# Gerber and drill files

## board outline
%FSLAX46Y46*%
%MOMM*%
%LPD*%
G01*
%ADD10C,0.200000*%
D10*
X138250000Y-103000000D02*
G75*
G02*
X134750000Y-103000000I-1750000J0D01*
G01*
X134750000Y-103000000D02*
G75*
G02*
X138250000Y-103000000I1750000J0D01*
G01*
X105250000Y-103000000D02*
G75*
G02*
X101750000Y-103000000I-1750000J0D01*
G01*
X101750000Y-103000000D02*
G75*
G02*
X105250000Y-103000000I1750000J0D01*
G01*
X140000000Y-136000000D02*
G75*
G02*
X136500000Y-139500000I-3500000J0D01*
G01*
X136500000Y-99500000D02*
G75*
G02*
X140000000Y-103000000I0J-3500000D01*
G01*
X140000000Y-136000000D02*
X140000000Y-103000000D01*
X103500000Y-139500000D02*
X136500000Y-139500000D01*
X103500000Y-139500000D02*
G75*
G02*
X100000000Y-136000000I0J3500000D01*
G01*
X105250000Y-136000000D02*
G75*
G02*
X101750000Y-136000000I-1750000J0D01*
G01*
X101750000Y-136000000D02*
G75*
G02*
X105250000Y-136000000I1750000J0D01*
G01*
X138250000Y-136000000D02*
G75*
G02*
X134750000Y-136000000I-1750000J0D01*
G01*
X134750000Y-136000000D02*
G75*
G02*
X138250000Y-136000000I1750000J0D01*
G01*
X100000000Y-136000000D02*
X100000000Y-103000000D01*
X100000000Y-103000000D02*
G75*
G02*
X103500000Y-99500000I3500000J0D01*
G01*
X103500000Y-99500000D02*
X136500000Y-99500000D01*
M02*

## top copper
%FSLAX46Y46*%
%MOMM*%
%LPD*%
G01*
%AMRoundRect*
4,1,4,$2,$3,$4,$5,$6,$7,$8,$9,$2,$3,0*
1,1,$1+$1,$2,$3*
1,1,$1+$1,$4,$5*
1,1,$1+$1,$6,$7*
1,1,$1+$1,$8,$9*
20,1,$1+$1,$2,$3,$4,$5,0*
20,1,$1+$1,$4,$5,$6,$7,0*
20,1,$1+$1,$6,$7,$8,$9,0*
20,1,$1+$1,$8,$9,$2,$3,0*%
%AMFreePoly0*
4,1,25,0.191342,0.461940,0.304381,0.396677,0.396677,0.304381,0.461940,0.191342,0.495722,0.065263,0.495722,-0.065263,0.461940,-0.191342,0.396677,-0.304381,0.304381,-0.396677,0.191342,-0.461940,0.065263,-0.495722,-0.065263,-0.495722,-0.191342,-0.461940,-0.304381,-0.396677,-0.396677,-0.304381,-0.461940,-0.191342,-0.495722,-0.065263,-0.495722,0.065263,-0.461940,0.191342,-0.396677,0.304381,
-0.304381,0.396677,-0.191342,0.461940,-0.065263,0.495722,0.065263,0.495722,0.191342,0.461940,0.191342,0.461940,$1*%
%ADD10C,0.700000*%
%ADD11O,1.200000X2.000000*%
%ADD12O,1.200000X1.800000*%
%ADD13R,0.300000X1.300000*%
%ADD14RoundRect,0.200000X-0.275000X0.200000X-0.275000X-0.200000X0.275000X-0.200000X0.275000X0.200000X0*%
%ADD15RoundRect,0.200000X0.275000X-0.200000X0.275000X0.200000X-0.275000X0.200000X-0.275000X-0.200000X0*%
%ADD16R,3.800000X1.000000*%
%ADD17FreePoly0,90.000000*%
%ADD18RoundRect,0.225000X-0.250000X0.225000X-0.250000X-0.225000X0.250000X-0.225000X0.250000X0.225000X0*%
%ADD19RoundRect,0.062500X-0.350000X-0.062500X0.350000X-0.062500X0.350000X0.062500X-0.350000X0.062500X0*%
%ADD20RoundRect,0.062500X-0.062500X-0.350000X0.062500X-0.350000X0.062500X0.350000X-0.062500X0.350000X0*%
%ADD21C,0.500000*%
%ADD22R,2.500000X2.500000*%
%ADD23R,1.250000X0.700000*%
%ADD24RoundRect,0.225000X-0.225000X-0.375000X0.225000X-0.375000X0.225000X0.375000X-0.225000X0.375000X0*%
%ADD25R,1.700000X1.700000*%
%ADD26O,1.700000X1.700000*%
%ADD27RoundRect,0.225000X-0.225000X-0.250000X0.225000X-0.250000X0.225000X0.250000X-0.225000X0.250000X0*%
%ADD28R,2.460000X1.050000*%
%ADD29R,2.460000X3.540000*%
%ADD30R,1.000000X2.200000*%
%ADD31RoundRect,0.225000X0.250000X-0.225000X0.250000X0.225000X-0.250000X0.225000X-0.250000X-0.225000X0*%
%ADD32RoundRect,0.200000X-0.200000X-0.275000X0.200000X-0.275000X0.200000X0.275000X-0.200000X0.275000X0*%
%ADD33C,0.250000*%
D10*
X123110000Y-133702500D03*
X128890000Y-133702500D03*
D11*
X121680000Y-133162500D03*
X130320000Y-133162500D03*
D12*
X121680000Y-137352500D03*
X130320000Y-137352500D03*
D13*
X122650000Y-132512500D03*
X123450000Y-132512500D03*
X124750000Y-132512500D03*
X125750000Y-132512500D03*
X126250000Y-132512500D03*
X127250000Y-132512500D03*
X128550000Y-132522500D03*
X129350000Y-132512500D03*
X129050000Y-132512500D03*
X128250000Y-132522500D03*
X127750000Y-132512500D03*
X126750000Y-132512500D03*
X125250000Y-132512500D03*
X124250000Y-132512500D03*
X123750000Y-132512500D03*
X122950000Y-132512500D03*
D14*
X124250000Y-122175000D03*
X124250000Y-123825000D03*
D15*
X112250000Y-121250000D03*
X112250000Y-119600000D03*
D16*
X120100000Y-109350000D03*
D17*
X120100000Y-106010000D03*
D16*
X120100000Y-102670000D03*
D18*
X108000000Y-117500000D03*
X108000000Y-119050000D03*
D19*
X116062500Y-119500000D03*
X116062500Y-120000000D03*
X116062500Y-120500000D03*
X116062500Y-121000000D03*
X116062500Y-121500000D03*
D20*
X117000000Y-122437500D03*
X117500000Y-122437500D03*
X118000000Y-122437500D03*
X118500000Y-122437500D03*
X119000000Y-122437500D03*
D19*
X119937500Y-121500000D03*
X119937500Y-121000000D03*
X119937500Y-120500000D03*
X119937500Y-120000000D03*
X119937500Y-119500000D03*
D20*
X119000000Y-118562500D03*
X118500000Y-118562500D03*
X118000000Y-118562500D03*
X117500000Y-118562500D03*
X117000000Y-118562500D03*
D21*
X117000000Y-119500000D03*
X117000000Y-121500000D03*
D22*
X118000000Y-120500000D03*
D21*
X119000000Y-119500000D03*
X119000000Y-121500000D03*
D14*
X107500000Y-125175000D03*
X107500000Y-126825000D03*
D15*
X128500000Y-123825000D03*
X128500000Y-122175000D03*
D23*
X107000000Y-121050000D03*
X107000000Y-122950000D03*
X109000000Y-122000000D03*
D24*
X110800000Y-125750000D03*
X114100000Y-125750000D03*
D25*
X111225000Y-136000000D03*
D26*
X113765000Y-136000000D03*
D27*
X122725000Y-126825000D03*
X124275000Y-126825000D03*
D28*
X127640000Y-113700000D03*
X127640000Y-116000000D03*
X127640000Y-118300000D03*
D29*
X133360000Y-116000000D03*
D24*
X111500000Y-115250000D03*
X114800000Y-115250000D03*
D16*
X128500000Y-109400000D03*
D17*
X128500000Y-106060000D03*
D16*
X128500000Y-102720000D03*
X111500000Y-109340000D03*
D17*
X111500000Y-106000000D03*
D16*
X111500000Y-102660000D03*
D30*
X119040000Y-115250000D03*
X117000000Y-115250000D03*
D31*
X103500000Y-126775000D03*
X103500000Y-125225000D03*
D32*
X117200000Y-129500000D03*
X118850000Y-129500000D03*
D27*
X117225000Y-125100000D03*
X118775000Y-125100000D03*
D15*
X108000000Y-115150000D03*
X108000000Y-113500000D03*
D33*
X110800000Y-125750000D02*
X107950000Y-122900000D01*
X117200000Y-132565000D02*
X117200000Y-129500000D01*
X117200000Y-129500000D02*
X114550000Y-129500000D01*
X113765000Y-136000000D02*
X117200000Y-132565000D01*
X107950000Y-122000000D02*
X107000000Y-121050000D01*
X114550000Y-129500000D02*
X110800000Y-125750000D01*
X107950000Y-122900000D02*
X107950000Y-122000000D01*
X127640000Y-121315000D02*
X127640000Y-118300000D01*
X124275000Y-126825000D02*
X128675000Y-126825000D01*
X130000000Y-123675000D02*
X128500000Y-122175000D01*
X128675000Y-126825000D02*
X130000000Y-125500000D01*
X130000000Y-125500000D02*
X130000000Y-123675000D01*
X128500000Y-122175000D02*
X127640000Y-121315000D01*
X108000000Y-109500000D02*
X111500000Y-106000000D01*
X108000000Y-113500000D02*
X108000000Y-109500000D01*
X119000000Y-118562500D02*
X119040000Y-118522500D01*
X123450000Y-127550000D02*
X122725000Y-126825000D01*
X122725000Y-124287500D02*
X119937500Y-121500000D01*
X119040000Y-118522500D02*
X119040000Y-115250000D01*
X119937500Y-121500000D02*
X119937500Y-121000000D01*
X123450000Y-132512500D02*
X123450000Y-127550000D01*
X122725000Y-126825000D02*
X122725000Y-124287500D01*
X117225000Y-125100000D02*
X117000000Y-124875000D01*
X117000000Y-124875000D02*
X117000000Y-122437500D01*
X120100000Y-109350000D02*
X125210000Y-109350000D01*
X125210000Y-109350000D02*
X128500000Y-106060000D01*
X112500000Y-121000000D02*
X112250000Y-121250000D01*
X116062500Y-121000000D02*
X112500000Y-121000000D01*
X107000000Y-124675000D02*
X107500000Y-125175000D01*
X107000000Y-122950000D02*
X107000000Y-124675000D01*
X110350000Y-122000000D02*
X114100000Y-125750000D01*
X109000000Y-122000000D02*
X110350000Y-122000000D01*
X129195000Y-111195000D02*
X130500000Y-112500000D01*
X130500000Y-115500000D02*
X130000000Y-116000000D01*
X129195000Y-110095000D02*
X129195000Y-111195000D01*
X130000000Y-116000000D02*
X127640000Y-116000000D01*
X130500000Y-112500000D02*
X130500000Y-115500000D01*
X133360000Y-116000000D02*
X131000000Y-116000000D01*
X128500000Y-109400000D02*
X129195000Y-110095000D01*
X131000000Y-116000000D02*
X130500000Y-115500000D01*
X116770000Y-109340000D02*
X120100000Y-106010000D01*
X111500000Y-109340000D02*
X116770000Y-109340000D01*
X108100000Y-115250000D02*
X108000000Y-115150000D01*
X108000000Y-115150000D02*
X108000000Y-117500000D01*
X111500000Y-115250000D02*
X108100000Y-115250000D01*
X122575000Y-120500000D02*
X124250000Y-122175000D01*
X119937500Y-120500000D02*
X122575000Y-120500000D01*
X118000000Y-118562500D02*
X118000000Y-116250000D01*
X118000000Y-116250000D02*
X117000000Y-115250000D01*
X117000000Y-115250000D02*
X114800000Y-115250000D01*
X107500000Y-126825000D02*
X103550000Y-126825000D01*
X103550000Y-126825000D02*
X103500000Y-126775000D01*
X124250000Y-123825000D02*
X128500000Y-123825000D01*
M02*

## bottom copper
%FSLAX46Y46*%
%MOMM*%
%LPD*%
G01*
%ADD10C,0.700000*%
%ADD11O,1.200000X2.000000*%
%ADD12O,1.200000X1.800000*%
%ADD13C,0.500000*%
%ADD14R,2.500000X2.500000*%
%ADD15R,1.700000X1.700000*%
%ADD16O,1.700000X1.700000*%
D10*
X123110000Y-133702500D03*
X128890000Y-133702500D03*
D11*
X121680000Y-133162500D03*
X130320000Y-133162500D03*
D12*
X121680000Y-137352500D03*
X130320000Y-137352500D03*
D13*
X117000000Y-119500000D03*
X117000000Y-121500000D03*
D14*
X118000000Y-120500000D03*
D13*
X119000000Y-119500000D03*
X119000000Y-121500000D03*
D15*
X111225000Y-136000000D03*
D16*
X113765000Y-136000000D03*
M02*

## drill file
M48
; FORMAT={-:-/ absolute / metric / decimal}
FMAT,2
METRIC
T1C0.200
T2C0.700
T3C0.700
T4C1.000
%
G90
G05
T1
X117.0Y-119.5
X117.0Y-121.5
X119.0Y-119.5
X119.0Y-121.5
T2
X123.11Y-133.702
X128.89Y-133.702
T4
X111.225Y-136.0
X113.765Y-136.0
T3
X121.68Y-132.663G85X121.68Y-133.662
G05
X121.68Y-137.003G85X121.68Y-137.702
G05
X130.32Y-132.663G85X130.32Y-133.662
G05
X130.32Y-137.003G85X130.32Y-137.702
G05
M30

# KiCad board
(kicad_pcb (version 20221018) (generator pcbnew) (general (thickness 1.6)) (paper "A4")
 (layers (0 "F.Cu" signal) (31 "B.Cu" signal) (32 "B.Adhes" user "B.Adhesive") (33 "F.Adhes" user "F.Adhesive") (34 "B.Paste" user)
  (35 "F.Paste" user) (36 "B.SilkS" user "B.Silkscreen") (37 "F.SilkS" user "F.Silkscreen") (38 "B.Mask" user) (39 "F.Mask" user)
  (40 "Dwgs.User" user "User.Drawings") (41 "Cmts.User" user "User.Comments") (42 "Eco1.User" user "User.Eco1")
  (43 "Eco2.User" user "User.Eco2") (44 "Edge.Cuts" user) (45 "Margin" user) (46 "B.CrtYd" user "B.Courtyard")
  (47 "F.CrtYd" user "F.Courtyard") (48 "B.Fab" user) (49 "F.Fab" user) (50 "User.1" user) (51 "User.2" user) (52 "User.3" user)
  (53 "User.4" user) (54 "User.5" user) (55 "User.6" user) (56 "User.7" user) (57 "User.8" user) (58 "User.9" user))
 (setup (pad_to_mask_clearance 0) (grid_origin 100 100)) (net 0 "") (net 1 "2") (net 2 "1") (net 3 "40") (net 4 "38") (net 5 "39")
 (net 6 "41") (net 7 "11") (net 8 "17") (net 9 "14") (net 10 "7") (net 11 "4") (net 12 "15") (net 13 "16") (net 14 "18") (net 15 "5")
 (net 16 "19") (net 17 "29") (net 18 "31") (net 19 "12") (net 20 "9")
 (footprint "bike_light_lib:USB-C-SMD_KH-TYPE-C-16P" (layer "F.Cu") (at 126 134.9325)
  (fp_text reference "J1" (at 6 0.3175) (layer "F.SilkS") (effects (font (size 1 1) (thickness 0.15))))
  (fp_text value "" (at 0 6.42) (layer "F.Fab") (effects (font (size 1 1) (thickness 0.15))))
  (pad "" thru_hole circle (at -2.89 -1.23) (size 0.7 0.7) (drill 0.7) (layers "*.Cu" "*.Mask"))
  (pad "" thru_hole circle (at 2.89 -1.23) (size 0.7 0.7) (drill 0.7) (layers "*.Cu" "*.Mask"))
  (pad "1" thru_hole oval (at -4.32 -1.77) (size 1.2 2) (drill oval 0.700024 1.699997) (layers "*.Cu" "*.Paste" "*.Mask") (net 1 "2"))
  (pad "2" thru_hole oval (at 4.32 -1.77) (size 1.2 2) (drill oval 0.700024 1.699997) (layers "*.Cu" "*.Paste" "*.Mask") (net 1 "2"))
  (pad "3" thru_hole oval (at -4.32 2.42) (size 1.2 1.8) (drill oval 0.700024 1.399997) (layers "*.Cu" "*.Paste" "*.Mask") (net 1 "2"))
  (pad "4" thru_hole oval (at 4.32 2.42) (size 1.2 1.8) (drill oval 0.700024 1.399997) (layers "*.Cu" "*.Paste" "*.Mask") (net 1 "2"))
  (pad "A1" smd rect (at -3.35 -2.42) (size 0.3 1.3) (layers "F.Cu" "F.Paste" "F.Mask") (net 1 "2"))
  (pad "A4" smd rect (at -2.55 -2.42) (size 0.3 1.3) (layers "F.Cu" "F.Paste" "F.Mask") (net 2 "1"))
  (pad "A5" smd rect (at -1.25 -2.42) (size 0.3 1.3) (layers "F.Cu" "F.Paste" "F.Mask") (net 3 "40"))
  (pad "A6" smd rect (at -0.25 -2.42) (size 0.3 1.3) (layers "F.Cu" "F.Paste" "F.Mask") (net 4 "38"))
  (pad "A7" smd rect (at 0.25 -2.42) (size 0.3 1.3) (layers "F.Cu" "F.Paste" "F.Mask") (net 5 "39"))
  (pad "A8" smd rect (at 1.25 -2.42) (size 0.3 1.3) (layers "F.Cu" "F.Paste" "F.Mask") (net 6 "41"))
  (pad "A9" smd rect (at 2.55 -2.41) (size 0.3 1.3) (layers "F.Cu" "F.Paste" "F.Mask") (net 2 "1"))
  (pad "A12" smd rect (at 3.35 -2.42) (size 0.3 1.3) (layers "F.Cu" "F.Paste" "F.Mask") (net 1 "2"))
  (pad "B1" smd rect (at 3.05 -2.42) (size 0.3 1.3) (layers "F.Cu" "F.Paste" "F.Mask") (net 1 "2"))
  (pad "B4" smd rect (at 2.25 -2.41) (size 0.3 1.3) (layers "F.Cu" "F.Paste" "F.Mask") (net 2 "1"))
  (pad "B5" smd rect (at 1.75 -2.42) (size 0.3 1.3) (layers "F.Cu" "F.Paste" "F.Mask") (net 3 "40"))
  (pad "B6" smd rect (at 0.75 -2.42) (size 0.3 1.3) (layers "F.Cu" "F.Paste" "F.Mask") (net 4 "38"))
  (pad "B7" smd rect (at -0.75 -2.42) (size 0.3 1.3) (layers "F.Cu" "F.Paste" "F.Mask") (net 5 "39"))
  (pad "B8" smd rect (at -1.75 -2.42) (size 0.3 1.3) (layers "F.Cu" "F.Paste" "F.Mask") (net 6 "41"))
  (pad "B9" smd rect (at -2.25 -2.42) (size 0.3 1.3) (layers "F.Cu" "F.Paste" "F.Mask") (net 2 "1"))
  (pad "B12" smd rect (at -3.05 -2.42) (size 0.3 1.3) (layers "F.Cu" "F.Paste" "F.Mask") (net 1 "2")))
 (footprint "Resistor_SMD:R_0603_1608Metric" (layer "F.Cu") (at 124.25 123 -90)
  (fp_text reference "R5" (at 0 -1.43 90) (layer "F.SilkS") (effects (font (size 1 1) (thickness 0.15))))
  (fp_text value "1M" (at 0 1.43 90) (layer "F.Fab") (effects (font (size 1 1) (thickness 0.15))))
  (pad "1" smd roundrect (at -0.825 0 270) (size 0.8 0.95) (layers "F.Cu" "F.Paste" "F.Mask") (roundrect_rratio 0.25) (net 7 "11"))
  (pad "2" smd roundrect (at 0.825 0 270) (size 0.8 0.95) (layers "F.Cu" "F.Paste" "F.Mask") (roundrect_rratio 0.25) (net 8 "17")))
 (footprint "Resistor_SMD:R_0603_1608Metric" (layer "F.Cu") (at 112.25 120.425 90)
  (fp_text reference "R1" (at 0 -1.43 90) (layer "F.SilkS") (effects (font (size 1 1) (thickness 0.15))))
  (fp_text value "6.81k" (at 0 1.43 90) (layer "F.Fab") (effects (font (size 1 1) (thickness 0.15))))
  (pad "1" smd roundrect (at -0.825 0 90) (size 0.8 0.95) (layers "F.Cu" "F.Paste" "F.Mask") (roundrect_rratio 0.25) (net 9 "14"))
  (pad "2" smd roundrect (at 0.825 0 90) (size 0.8 0.95) (layers "F.Cu" "F.Paste" "F.Mask") (roundrect_rratio 0.25) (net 1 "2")))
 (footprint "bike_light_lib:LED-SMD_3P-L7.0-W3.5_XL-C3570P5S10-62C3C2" (layer "F.Cu") (at 120.1 106.01 90)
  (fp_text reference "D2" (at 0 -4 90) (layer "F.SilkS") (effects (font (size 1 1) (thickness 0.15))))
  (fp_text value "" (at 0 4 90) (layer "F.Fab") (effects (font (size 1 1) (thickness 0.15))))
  (pad "1" smd rect (at -3.34 0 90) (size 1 3.8) (layers "F.Cu" "F.Paste" "F.Mask") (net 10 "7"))
  (pad "2" smd custom (at 0 0 90) (size 1 1) (layers "F.Cu" "F.Paste" "F.Mask") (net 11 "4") (thermal_bridge_angle 45)
   (options (clearance outline) (anchor circle)) (primitives))
  (pad "3" smd rect (at 3.34 0 90) (size 1 3.8) (layers "F.Cu" "F.Paste" "F.Mask")))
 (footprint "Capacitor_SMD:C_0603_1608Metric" (layer "F.Cu") (at 108 118.275 -90)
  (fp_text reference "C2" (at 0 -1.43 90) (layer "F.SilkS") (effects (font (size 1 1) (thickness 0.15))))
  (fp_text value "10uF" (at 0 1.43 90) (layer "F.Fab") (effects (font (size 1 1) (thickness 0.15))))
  (pad "1" smd roundrect (at -0.775 0 270) (size 0.9 0.95) (layers "F.Cu" "F.Paste" "F.Mask") (roundrect_rratio 0.25) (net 7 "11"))
  (pad "2" smd roundrect (at 0.775 0 270) (size 0.9 0.95) (layers "F.Cu" "F.Paste" "F.Mask") (roundrect_rratio 0.25) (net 1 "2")))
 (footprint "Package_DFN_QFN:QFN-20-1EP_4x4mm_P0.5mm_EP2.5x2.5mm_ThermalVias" (layer "F.Cu") (at 118 120.5)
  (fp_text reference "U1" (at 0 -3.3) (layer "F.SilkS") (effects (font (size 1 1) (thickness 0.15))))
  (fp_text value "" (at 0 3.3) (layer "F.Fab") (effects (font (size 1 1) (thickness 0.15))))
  (pad "" smd roundrect (at -0.625 -0.625) (size 1.08 1.08) (layers "F.Paste") (roundrect_rratio 0.231481))
  (pad "" smd roundrect (at -0.625 0.625) (size 1.08 1.08) (layers "F.Paste") (roundrect_rratio 0.231481))
  (pad "" smd roundrect (at 0.625 -0.625) (size 1.08 1.08) (layers "F.Paste") (roundrect_rratio 0.231481))
  (pad "" smd roundrect (at 0.625 0.625) (size 1.08 1.08) (layers "F.Paste") (roundrect_rratio 0.231481))
  (pad "1" smd roundrect (at -1.9375 -1) (size 0.825 0.25) (layers "F.Cu" "F.Paste" "F.Mask") (roundrect_rratio 0.25))
  (pad "2" smd roundrect (at -1.9375 -0.5) (size 0.825 0.25) (layers "F.Cu" "F.Paste" "F.Mask") (roundrect_rratio 0.25))
  (pad "3" smd roundrect (at -1.9375 0) (size 0.825 0.25) (layers "F.Cu" "F.Paste" "F.Mask") (roundrect_rratio 0.25) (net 2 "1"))
  (pad "4" smd roundrect (at -1.9375 0.5) (size 0.825 0.25) (layers "F.Cu" "F.Paste" "F.Mask") (roundrect_rratio 0.25) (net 9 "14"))
  (pad "5" smd roundrect (at -1.9375 1) (size 0.825 0.25) (layers "F.Cu" "F.Paste" "F.Mask") (roundrect_rratio 0.25) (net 2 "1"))
  (pad "6" smd roundrect (at -1 1.9375) (size 0.25 0.825) (layers "F.Cu" "F.Paste" "F.Mask") (roundrect_rratio 0.25) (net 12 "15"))
  (pad "7" smd roundrect (at -0.5 1.9375) (size 0.25 0.825) (layers "F.Cu" "F.Paste" "F.Mask") (roundrect_rratio 0.25) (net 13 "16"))
  (pad "8" smd roundrect (at 0 1.9375) (size 0.25 0.825) (layers "F.Cu" "F.Paste" "F.Mask") (roundrect_rratio 0.25) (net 8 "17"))
  (pad "9" smd roundrect (at 0.5 1.9375) (size 0.25 0.825) (layers "F.Cu" "F.Paste" "F.Mask") (roundrect_rratio 0.25) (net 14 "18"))
  (pad "10" smd roundrect (at 1 1.9375) (size 0.25 0.825) (layers "F.Cu" "F.Paste" "F.Mask") (roundrect_rratio 0.25) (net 14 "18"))
  (pad "11" smd roundrect (at 1.9375 1) (size 0.825 0.25) (layers "F.Cu" "F.Paste" "F.Mask") (roundrect_rratio 0.25) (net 2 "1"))
  (pad "12" smd roundrect (at 1.9375 0.5) (size 0.825 0.25) (layers "F.Cu" "F.Paste" "F.Mask") (roundrect_rratio 0.25) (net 2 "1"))
  (pad "13" smd roundrect (at 1.9375 0) (size 0.825 0.25) (layers "F.Cu" "F.Paste" "F.Mask") (roundrect_rratio 0.25) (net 7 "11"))
  (pad "14" smd roundrect (at 1.9375 -0.5) (size 0.825 0.25) (layers "F.Cu" "F.Paste" "F.Mask") (roundrect_rratio 0.25) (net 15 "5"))
  (pad "15" smd roundrect (at 1.9375 -1) (size 0.825 0.25) (layers "F.Cu" "F.Paste" "F.Mask") (roundrect_rratio 0.25) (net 2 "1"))
  (pad "16" smd roundrect (at 1 -1.9375) (size 0.25 0.825) (layers "F.Cu" "F.Paste" "F.Mask") (roundrect_rratio 0.25) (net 2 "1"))
  (pad "17" smd roundrect (at 0.5 -1.9375) (size 0.25 0.825) (layers "F.Cu" "F.Paste" "F.Mask") (roundrect_rratio 0.25) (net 1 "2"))
  (pad "18" smd roundrect (at 0 -1.9375) (size 0.25 0.825) (layers "F.Cu" "F.Paste" "F.Mask") (roundrect_rratio 0.25) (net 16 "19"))
  (pad "19" smd roundrect (at -0.5 -1.9375) (size 0.25 0.825) (layers "F.Cu" "F.Paste" "F.Mask") (roundrect_rratio 0.25))
  (pad "20" smd roundrect (at -1 -1.9375) (size 0.25 0.825) (layers "F.Cu" "F.Paste" "F.Mask") (roundrect_rratio 0.25))
  (pad "21" thru_hole circle (at -1 -1) (size 0.5 0.5) (drill 0.2) (layers "*.Cu"))
  (pad "21" thru_hole circle (at -1 1) (size 0.5 0.5) (drill 0.2) (layers "*.Cu"))
  (pad "21" smd rect (at 0 0) (size 2.5 2.5) (layers "F.Cu" "F.Mask")) (pad "21" smd rect (at 0 0) (size 2.5 2.5) (layers "B.Cu"))
  (pad "21" thru_hole circle (at 1 -1) (size 0.5 0.5) (drill 0.2) (layers "*.Cu"))
  (pad "21" thru_hole circle (at 1 1) (size 0.5 0.5) (drill 0.2) (layers "*.Cu")))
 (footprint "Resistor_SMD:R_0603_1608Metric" (layer "F.Cu") (at 107.5 126 -90)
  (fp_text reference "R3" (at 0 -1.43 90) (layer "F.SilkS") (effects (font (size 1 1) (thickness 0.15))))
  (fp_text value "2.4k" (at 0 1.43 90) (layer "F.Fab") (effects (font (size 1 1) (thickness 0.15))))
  (pad "1" smd roundrect (at -0.825 0 270) (size 0.8 0.95) (layers "F.Cu" "F.Paste" "F.Mask") (roundrect_rratio 0.25) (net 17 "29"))
  (pad "2" smd roundrect (at 0.825 0 270) (size 0.8 0.95) (layers "F.Cu" "F.Paste" "F.Mask") (roundrect_rratio 0.25) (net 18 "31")))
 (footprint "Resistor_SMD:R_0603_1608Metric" (layer "F.Cu") (at 128.5 123 90)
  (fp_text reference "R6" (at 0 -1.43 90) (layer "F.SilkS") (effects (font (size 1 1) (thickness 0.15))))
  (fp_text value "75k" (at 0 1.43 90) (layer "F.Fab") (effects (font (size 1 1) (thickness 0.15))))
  (pad "1" smd roundrect (at -0.825 0 90) (size 0.8 0.95) (layers "F.Cu" "F.Paste" "F.Mask") (roundrect_rratio 0.25) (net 8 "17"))
  (pad "2" smd roundrect (at 0.825 0 90) (size 0.8 0.95) (layers "F.Cu" "F.Paste" "F.Mask") (roundrect_rratio 0.25) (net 1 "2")))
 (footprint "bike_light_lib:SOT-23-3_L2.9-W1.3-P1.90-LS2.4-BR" (layer "F.Cu") (at 108 122 180)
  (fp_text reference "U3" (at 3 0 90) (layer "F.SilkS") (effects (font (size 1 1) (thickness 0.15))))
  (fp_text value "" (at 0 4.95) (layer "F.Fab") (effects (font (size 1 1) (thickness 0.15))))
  (pad "1" smd rect (at 1 0.95 180) (size 1.25 0.7) (layers "F.Cu" "F.Paste" "F.Mask") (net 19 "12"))
  (pad "2" smd rect (at 1 -0.95 180) (size 1.25 0.7) (layers "F.Cu" "F.Paste" "F.Mask") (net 17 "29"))
  (pad "3" smd rect (at -1 0 180) (size 1.25 0.7) (layers "F.Cu" "F.Paste" "F.Mask") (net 13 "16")))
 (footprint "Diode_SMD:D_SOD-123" (layer "F.Cu") (at 112.45 125.75)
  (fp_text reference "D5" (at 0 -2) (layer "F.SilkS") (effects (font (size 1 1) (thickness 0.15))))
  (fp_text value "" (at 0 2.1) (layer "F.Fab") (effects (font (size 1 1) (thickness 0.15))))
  (pad "1" smd roundrect (at -1.65 0) (size 0.9 1.2) (layers "F.Cu" "F.Paste" "F.Mask") (roundrect_rratio 0.25) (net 19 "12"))
  (pad "2" smd roundrect (at 1.65 0) (size 0.9 1.2) (layers "F.Cu" "F.Paste" "F.Mask") (roundrect_rratio 0.25) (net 13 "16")))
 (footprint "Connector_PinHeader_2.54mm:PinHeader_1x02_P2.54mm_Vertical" (layer "F.Cu") (at 111.225 136 90)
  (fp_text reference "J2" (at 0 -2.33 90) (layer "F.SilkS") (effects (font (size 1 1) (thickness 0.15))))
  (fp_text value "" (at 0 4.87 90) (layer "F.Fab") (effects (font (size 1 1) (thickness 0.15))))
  (pad "1" thru_hole rect (at 0 0 90) (size 1.7 1.7) (drill 1) (layers "*.Cu" "*.Mask") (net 1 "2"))
  (pad "2" thru_hole oval (at 0 2.54 90) (size 1.7 1.7) (drill 1) (layers "*.Cu" "*.Mask") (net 19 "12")))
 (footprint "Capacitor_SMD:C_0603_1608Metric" (layer "F.Cu") (at 123.5 126.825)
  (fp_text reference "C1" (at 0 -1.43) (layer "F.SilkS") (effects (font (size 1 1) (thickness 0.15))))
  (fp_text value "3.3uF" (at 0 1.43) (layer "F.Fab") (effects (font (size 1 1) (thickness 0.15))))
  (pad "1" smd roundrect (at -0.775 0) (size 0.9 0.95) (layers "F.Cu" "F.Paste" "F.Mask") (roundrect_rratio 0.25) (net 2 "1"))
  (pad "2" smd roundrect (at 0.775 0) (size 0.9 0.95) (layers "F.Cu" "F.Paste" "F.Mask") (roundrect_rratio 0.25) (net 1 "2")))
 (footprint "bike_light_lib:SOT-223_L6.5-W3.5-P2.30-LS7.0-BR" (layer "F.Cu") (at 130.5 116 180)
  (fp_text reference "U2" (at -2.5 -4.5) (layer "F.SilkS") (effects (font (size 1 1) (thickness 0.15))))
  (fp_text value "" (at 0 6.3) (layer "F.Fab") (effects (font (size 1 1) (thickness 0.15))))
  (pad "1" smd rect (at 2.86 2.3 180) (size 2.46 1.05) (layers "F.Cu" "F.Paste" "F.Mask") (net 19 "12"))
  (pad "2" smd rect (at 2.86 0 180) (size 2.46 1.05) (layers "F.Cu" "F.Paste" "F.Mask") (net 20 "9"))
  (pad "3" smd rect (at 2.86 -2.3 180) (size 2.46 1.05) (layers "F.Cu" "F.Paste" "F.Mask") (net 1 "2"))
  (pad "4" smd rect (at -2.86 0 180) (size 2.46 3.54) (layers "F.Cu" "F.Paste" "F.Mask") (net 20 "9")))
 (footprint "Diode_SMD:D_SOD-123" (layer "F.Cu") (at 113.15 115.25)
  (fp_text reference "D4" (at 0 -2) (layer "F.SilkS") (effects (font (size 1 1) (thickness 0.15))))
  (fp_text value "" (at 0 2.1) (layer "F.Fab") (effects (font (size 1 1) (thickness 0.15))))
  (pad "1" smd roundrect (at -1.65 0) (size 0.9 1.2) (layers "F.Cu" "F.Paste" "F.Mask") (roundrect_rratio 0.25) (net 7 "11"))
  (pad "2" smd roundrect (at 1.65 0) (size 0.9 1.2) (layers "F.Cu" "F.Paste" "F.Mask") (roundrect_rratio 0.25) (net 16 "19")))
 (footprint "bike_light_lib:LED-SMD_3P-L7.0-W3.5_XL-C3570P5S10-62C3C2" (layer "F.Cu") (at 128.5 106.06 90)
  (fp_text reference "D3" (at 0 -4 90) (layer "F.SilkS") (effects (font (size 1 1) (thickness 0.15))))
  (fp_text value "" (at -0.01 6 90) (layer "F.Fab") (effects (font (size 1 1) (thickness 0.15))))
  (pad "1" smd rect (at -3.34 0 90) (size 1 3.8) (layers "F.Cu" "F.Paste" "F.Mask") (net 20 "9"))
  (pad "2" smd custom (at 0 0 90) (size 1 1) (layers "F.Cu" "F.Paste" "F.Mask") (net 10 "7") (thermal_bridge_angle 45)
   (options (clearance outline) (anchor circle)) (primitives))
  (pad "3" smd rect (at 3.34 0 90) (size 1 3.8) (layers "F.Cu" "F.Paste" "F.Mask")))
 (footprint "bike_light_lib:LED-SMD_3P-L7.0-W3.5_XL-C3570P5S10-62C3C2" (layer "F.Cu") (at 111.5 106 90)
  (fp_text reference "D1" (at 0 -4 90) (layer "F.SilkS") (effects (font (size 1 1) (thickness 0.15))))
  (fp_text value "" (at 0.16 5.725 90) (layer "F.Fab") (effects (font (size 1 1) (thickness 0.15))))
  (pad "1" smd rect (at -3.34 0 90) (size 1 3.8) (layers "F.Cu" "F.Paste" "F.Mask") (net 11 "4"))
  (pad "2" smd custom (at 0 0 90) (size 1 1) (layers "F.Cu" "F.Paste" "F.Mask") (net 15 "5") (thermal_bridge_angle 45)
   (options (clearance outline) (anchor circle)) (primitives))
  (pad "3" smd rect (at 3.34 0 90) (size 1 3.8) (layers "F.Cu" "F.Paste" "F.Mask")))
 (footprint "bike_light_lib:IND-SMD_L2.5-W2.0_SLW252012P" (layer "F.Cu") (at 118.02 115.25 180)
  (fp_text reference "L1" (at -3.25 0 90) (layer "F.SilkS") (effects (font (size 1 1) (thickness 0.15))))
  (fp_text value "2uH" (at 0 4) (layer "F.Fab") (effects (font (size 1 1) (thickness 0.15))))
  (pad "1" smd rect (at -1.02 0 180) (size 1 2.2) (layers "F.Cu" "F.Paste" "F.Mask") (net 2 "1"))
  (pad "2" smd rect (at 1.02 0 180) (size 1 2.2) (layers "F.Cu" "F.Paste" "F.Mask") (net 16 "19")))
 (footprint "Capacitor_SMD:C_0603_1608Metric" (layer "F.Cu") (at 103.5 126 90)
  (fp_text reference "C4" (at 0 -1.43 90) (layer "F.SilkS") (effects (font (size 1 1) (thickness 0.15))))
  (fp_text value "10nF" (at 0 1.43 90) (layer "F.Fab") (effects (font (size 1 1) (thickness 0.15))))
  (pad "1" smd roundrect (at -0.775 0 90) (size 0.9 0.95) (layers "F.Cu" "F.Paste" "F.Mask") (roundrect_rratio 0.25) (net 18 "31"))
  (pad "2" smd roundrect (at 0.775 0 90) (size 0.9 0.95) (layers "F.Cu" "F.Paste" "F.Mask") (roundrect_rratio 0.25) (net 1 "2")))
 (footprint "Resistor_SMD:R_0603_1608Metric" (layer "F.Cu") (at 118.025 129.5)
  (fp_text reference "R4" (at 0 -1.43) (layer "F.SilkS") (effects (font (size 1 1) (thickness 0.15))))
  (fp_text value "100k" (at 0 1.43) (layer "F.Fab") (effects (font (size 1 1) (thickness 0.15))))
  (pad "1" smd roundrect (at -0.825 0) (size 0.8 0.95) (layers "F.Cu" "F.Paste" "F.Mask") (roundrect_rratio 0.25) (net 19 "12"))
  (pad "2" smd roundrect (at 0.825 0) (size 0.8 0.95) (layers "F.Cu" "F.Paste" "F.Mask") (roundrect_rratio 0.25) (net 1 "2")))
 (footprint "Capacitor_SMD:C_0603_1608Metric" (layer "F.Cu") (at 118 125.1)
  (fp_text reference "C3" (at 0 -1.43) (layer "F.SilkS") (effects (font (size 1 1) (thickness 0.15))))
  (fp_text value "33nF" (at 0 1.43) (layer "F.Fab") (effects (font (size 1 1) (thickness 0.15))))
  (pad "1" smd roundrect (at -0.775 0) (size 0.9 0.95) (layers "F.Cu" "F.Paste" "F.Mask") (roundrect_rratio 0.25) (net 12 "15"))
  (pad "2" smd roundrect (at 0.775 0) (size 0.9 0.95) (layers "F.Cu" "F.Paste" "F.Mask") (roundrect_rratio 0.25) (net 1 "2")))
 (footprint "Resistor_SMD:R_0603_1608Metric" (layer "F.Cu") (at 108 114.325 90)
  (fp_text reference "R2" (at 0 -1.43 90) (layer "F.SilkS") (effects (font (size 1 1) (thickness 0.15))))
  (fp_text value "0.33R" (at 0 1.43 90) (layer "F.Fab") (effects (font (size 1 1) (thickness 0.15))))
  (pad "1" smd roundrect (at -0.825 0 90) (size 0.8 0.95) (layers "F.Cu" "F.Paste" "F.Mask") (roundrect_rratio 0.25) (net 7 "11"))
  (pad "2" smd roundrect (at 0.825 0 90) (size 0.8 0.95) (layers "F.Cu" "F.Paste" "F.Mask") (roundrect_rratio 0.25) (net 15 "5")))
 (gr_circle (center 136.5 103) (end 138.25 103) (stroke (width 0.2) (type solid)) (fill none) (layer "Edge.Cuts"))
 (gr_circle (center 103.5 103) (end 105.25 103) (stroke (width 0.2) (type solid)) (fill none) (layer "Edge.Cuts"))
 (gr_arc (start 140 136) (mid 138.974874 138.474874) (end 136.5 139.5) (stroke (width 0.2) (type solid)) (layer "Edge.Cuts"))
 (gr_arc (start 136.5 99.5) (mid 138.974874 100.525126) (end 140 103) (stroke (width 0.2) (type solid)) (layer "Edge.Cuts"))
 (gr_line (start 140 136) (end 140 103) (stroke (width 0.2) (type solid)) (layer "Edge.Cuts"))
 (gr_line (start 103.5 139.5) (end 136.5 139.5) (stroke (width 0.2) (type solid)) (layer "Edge.Cuts"))
 (gr_arc (start 103.5 139.5) (mid 101.025126 138.474874) (end 100 136) (stroke (width 0.2) (type solid)) (layer "Edge.Cuts"))
 (gr_circle (center 103.5 136) (end 105.25 136) (stroke (width 0.2) (type solid)) (fill none) (layer "Edge.Cuts"))
 (gr_circle (center 136.5 136) (end 138.25 136) (stroke (width 0.2) (type solid)) (fill none) (layer "Edge.Cuts"))
 (gr_line (start 100 136) (end 100 103) (stroke (width 0.2) (type solid)) (layer "Edge.Cuts"))
 (gr_arc (start 100 103) (mid 101.025126 100.525126) (end 103.5 99.5) (stroke (width 0.2) (type solid)) (layer "Edge.Cuts"))
 (gr_line (start 103.5 99.5) (end 136.5 99.5) (stroke (width 0.2) (type solid)) (layer "Edge.Cuts"))
 (segment (start 110.8 125.75) (end 107.95 122.9) (width 0.25) (layer "F.Cu") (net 19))
 (segment (start 117.2 132.565) (end 117.2 129.5) (width 0.25) (layer "F.Cu") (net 19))
 (segment (start 117.2 129.5) (end 114.55 129.5) (width 0.25) (layer "F.Cu") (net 19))
 (segment (start 113.765 136) (end 117.2 132.565) (width 0.25) (layer "F.Cu") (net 19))
 (segment (start 107.95 122) (end 107 121.05) (width 0.25) (layer "F.Cu") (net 19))
 (segment (start 114.55 129.5) (end 110.8 125.75) (width 0.25) (layer "F.Cu") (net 19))
 (segment (start 107.95 122.9) (end 107.95 122) (width 0.25) (layer "F.Cu") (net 19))
 (segment (start 127.64 121.315) (end 127.64 118.3) (width 0.25) (layer "F.Cu") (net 1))
 (segment (start 124.275 126.825) (end 128.675 126.825) (width 0.25) (layer "F.Cu") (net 1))
 (segment (start 130 123.675) (end 128.5 122.175) (width 0.25) (layer "F.Cu") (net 1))
 (segment (start 128.675 126.825) (end 130 125.5) (width 0.25) (layer "F.Cu") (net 1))
 (segment (start 130 125.5) (end 130 123.675) (width 0.25) (layer "F.Cu") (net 1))
 (segment (start 128.5 122.175) (end 127.64 121.315) (width 0.25) (layer "F.Cu") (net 1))
 (segment (start 108 109.5) (end 111.5 106) (width 0.25) (layer "F.Cu") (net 15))
 (segment (start 108 113.5) (end 108 109.5) (width 0.25) (layer "F.Cu") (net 15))
 (segment (start 119 118.5625) (end 119.04 118.5225) (width 0.25) (layer "F.Cu") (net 2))
 (segment (start 123.45 127.55) (end 122.725 126.825) (width 0.25) (layer "F.Cu") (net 2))
 (segment (start 122.725 124.2875) (end 119.9375 121.5) (width 0.25) (layer "F.Cu") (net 2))
 (segment (start 119.04 118.5225) (end 119.04 115.25) (width 0.25) (layer "F.Cu") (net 2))
 (segment (start 119.9375 121.5) (end 119.9375 121) (width 0.25) (layer "F.Cu") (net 2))
 (segment (start 123.45 132.5125) (end 123.45 127.55) (width 0.25) (layer "F.Cu") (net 2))
 (segment (start 122.725 126.825) (end 122.725 124.2875) (width 0.25) (layer "F.Cu") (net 2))
 (segment (start 117.225 125.1) (end 117 124.875) (width 0.25) (layer "F.Cu") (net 12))
 (segment (start 117 124.875) (end 117 122.4375) (width 0.25) (layer "F.Cu") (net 12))
 (segment (start 120.1 109.35) (end 125.21 109.35) (width 0.25) (layer "F.Cu") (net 10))
 (segment (start 125.21 109.35) (end 128.5 106.06) (width 0.25) (layer "F.Cu") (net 10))
 (segment (start 112.5 121) (end 112.25 121.25) (width 0.25) (layer "F.Cu") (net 9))
 (segment (start 116.0625 121) (end 112.5 121) (width 0.25) (layer "F.Cu") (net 9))
 (segment (start 107 124.675) (end 107.5 125.175) (width 0.25) (layer "F.Cu") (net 17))
 (segment (start 107 122.95) (end 107 124.675) (width 0.25) (layer "F.Cu") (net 17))
 (segment (start 110.35 122) (end 114.1 125.75) (width 0.25) (layer "F.Cu") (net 13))
 (segment (start 109 122) (end 110.35 122) (width 0.25) (layer "F.Cu") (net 13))
 (segment (start 129.195 111.195) (end 130.5 112.5) (width 0.25) (layer "F.Cu") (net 20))
 (segment (start 130.5 115.5) (end 130 116) (width 0.25) (layer "F.Cu") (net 20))
 (segment (start 129.195 110.095) (end 129.195 111.195) (width 0.25) (layer "F.Cu") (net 20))
 (segment (start 130 116) (end 127.64 116) (width 0.25) (layer "F.Cu") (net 20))
 (segment (start 130.5 112.5) (end 130.5 115.5) (width 0.25) (layer "F.Cu") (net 20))
 (segment (start 133.36 116) (end 131 116) (width 0.25) (layer "F.Cu") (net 20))
 (segment (start 128.5 109.4) (end 129.195 110.095) (width 0.25) (layer "F.Cu") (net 20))
 (segment (start 131 116) (end 130.5 115.5) (width 0.25) (layer "F.Cu") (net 20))
 (segment (start 116.77 109.34) (end 120.1 106.01) (width 0.25) (layer "F.Cu") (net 11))
 (segment (start 111.5 109.34) (end 116.77 109.34) (width 0.25) (layer "F.Cu") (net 11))
 (segment (start 108.1 115.25) (end 108 115.15) (width 0.25) (layer "F.Cu") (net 7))
 (segment (start 108 115.15) (end 108 117.5) (width 0.25) (layer "F.Cu") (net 7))
 (segment (start 111.5 115.25) (end 108.1 115.25) (width 0.25) (layer "F.Cu") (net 7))
 (segment (start 122.575 120.5) (end 124.25 122.175) (width 0.25) (layer "F.Cu") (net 7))
 (segment (start 119.9375 120.5) (end 122.575 120.5) (width 0.25) (layer "F.Cu") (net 7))
 (segment (start 118 118.5625) (end 118 116.25) (width 0.25) (layer "F.Cu") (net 16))
 (segment (start 118 116.25) (end 117 115.25) (width 0.25) (layer "F.Cu") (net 16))
 (segment (start 117 115.25) (end 114.8 115.25) (width 0.25) (layer "F.Cu") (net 16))
 (segment (start 107.5 126.825) (end 103.55 126.825) (width 0.25) (layer "F.Cu") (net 18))
 (segment (start 103.55 126.825) (end 103.5 126.775) (width 0.25) (layer "F.Cu") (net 18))
 (segment (start 124.25 123.825) (end 128.5 123.825) (width 0.25) (layer "F.Cu") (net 8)))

